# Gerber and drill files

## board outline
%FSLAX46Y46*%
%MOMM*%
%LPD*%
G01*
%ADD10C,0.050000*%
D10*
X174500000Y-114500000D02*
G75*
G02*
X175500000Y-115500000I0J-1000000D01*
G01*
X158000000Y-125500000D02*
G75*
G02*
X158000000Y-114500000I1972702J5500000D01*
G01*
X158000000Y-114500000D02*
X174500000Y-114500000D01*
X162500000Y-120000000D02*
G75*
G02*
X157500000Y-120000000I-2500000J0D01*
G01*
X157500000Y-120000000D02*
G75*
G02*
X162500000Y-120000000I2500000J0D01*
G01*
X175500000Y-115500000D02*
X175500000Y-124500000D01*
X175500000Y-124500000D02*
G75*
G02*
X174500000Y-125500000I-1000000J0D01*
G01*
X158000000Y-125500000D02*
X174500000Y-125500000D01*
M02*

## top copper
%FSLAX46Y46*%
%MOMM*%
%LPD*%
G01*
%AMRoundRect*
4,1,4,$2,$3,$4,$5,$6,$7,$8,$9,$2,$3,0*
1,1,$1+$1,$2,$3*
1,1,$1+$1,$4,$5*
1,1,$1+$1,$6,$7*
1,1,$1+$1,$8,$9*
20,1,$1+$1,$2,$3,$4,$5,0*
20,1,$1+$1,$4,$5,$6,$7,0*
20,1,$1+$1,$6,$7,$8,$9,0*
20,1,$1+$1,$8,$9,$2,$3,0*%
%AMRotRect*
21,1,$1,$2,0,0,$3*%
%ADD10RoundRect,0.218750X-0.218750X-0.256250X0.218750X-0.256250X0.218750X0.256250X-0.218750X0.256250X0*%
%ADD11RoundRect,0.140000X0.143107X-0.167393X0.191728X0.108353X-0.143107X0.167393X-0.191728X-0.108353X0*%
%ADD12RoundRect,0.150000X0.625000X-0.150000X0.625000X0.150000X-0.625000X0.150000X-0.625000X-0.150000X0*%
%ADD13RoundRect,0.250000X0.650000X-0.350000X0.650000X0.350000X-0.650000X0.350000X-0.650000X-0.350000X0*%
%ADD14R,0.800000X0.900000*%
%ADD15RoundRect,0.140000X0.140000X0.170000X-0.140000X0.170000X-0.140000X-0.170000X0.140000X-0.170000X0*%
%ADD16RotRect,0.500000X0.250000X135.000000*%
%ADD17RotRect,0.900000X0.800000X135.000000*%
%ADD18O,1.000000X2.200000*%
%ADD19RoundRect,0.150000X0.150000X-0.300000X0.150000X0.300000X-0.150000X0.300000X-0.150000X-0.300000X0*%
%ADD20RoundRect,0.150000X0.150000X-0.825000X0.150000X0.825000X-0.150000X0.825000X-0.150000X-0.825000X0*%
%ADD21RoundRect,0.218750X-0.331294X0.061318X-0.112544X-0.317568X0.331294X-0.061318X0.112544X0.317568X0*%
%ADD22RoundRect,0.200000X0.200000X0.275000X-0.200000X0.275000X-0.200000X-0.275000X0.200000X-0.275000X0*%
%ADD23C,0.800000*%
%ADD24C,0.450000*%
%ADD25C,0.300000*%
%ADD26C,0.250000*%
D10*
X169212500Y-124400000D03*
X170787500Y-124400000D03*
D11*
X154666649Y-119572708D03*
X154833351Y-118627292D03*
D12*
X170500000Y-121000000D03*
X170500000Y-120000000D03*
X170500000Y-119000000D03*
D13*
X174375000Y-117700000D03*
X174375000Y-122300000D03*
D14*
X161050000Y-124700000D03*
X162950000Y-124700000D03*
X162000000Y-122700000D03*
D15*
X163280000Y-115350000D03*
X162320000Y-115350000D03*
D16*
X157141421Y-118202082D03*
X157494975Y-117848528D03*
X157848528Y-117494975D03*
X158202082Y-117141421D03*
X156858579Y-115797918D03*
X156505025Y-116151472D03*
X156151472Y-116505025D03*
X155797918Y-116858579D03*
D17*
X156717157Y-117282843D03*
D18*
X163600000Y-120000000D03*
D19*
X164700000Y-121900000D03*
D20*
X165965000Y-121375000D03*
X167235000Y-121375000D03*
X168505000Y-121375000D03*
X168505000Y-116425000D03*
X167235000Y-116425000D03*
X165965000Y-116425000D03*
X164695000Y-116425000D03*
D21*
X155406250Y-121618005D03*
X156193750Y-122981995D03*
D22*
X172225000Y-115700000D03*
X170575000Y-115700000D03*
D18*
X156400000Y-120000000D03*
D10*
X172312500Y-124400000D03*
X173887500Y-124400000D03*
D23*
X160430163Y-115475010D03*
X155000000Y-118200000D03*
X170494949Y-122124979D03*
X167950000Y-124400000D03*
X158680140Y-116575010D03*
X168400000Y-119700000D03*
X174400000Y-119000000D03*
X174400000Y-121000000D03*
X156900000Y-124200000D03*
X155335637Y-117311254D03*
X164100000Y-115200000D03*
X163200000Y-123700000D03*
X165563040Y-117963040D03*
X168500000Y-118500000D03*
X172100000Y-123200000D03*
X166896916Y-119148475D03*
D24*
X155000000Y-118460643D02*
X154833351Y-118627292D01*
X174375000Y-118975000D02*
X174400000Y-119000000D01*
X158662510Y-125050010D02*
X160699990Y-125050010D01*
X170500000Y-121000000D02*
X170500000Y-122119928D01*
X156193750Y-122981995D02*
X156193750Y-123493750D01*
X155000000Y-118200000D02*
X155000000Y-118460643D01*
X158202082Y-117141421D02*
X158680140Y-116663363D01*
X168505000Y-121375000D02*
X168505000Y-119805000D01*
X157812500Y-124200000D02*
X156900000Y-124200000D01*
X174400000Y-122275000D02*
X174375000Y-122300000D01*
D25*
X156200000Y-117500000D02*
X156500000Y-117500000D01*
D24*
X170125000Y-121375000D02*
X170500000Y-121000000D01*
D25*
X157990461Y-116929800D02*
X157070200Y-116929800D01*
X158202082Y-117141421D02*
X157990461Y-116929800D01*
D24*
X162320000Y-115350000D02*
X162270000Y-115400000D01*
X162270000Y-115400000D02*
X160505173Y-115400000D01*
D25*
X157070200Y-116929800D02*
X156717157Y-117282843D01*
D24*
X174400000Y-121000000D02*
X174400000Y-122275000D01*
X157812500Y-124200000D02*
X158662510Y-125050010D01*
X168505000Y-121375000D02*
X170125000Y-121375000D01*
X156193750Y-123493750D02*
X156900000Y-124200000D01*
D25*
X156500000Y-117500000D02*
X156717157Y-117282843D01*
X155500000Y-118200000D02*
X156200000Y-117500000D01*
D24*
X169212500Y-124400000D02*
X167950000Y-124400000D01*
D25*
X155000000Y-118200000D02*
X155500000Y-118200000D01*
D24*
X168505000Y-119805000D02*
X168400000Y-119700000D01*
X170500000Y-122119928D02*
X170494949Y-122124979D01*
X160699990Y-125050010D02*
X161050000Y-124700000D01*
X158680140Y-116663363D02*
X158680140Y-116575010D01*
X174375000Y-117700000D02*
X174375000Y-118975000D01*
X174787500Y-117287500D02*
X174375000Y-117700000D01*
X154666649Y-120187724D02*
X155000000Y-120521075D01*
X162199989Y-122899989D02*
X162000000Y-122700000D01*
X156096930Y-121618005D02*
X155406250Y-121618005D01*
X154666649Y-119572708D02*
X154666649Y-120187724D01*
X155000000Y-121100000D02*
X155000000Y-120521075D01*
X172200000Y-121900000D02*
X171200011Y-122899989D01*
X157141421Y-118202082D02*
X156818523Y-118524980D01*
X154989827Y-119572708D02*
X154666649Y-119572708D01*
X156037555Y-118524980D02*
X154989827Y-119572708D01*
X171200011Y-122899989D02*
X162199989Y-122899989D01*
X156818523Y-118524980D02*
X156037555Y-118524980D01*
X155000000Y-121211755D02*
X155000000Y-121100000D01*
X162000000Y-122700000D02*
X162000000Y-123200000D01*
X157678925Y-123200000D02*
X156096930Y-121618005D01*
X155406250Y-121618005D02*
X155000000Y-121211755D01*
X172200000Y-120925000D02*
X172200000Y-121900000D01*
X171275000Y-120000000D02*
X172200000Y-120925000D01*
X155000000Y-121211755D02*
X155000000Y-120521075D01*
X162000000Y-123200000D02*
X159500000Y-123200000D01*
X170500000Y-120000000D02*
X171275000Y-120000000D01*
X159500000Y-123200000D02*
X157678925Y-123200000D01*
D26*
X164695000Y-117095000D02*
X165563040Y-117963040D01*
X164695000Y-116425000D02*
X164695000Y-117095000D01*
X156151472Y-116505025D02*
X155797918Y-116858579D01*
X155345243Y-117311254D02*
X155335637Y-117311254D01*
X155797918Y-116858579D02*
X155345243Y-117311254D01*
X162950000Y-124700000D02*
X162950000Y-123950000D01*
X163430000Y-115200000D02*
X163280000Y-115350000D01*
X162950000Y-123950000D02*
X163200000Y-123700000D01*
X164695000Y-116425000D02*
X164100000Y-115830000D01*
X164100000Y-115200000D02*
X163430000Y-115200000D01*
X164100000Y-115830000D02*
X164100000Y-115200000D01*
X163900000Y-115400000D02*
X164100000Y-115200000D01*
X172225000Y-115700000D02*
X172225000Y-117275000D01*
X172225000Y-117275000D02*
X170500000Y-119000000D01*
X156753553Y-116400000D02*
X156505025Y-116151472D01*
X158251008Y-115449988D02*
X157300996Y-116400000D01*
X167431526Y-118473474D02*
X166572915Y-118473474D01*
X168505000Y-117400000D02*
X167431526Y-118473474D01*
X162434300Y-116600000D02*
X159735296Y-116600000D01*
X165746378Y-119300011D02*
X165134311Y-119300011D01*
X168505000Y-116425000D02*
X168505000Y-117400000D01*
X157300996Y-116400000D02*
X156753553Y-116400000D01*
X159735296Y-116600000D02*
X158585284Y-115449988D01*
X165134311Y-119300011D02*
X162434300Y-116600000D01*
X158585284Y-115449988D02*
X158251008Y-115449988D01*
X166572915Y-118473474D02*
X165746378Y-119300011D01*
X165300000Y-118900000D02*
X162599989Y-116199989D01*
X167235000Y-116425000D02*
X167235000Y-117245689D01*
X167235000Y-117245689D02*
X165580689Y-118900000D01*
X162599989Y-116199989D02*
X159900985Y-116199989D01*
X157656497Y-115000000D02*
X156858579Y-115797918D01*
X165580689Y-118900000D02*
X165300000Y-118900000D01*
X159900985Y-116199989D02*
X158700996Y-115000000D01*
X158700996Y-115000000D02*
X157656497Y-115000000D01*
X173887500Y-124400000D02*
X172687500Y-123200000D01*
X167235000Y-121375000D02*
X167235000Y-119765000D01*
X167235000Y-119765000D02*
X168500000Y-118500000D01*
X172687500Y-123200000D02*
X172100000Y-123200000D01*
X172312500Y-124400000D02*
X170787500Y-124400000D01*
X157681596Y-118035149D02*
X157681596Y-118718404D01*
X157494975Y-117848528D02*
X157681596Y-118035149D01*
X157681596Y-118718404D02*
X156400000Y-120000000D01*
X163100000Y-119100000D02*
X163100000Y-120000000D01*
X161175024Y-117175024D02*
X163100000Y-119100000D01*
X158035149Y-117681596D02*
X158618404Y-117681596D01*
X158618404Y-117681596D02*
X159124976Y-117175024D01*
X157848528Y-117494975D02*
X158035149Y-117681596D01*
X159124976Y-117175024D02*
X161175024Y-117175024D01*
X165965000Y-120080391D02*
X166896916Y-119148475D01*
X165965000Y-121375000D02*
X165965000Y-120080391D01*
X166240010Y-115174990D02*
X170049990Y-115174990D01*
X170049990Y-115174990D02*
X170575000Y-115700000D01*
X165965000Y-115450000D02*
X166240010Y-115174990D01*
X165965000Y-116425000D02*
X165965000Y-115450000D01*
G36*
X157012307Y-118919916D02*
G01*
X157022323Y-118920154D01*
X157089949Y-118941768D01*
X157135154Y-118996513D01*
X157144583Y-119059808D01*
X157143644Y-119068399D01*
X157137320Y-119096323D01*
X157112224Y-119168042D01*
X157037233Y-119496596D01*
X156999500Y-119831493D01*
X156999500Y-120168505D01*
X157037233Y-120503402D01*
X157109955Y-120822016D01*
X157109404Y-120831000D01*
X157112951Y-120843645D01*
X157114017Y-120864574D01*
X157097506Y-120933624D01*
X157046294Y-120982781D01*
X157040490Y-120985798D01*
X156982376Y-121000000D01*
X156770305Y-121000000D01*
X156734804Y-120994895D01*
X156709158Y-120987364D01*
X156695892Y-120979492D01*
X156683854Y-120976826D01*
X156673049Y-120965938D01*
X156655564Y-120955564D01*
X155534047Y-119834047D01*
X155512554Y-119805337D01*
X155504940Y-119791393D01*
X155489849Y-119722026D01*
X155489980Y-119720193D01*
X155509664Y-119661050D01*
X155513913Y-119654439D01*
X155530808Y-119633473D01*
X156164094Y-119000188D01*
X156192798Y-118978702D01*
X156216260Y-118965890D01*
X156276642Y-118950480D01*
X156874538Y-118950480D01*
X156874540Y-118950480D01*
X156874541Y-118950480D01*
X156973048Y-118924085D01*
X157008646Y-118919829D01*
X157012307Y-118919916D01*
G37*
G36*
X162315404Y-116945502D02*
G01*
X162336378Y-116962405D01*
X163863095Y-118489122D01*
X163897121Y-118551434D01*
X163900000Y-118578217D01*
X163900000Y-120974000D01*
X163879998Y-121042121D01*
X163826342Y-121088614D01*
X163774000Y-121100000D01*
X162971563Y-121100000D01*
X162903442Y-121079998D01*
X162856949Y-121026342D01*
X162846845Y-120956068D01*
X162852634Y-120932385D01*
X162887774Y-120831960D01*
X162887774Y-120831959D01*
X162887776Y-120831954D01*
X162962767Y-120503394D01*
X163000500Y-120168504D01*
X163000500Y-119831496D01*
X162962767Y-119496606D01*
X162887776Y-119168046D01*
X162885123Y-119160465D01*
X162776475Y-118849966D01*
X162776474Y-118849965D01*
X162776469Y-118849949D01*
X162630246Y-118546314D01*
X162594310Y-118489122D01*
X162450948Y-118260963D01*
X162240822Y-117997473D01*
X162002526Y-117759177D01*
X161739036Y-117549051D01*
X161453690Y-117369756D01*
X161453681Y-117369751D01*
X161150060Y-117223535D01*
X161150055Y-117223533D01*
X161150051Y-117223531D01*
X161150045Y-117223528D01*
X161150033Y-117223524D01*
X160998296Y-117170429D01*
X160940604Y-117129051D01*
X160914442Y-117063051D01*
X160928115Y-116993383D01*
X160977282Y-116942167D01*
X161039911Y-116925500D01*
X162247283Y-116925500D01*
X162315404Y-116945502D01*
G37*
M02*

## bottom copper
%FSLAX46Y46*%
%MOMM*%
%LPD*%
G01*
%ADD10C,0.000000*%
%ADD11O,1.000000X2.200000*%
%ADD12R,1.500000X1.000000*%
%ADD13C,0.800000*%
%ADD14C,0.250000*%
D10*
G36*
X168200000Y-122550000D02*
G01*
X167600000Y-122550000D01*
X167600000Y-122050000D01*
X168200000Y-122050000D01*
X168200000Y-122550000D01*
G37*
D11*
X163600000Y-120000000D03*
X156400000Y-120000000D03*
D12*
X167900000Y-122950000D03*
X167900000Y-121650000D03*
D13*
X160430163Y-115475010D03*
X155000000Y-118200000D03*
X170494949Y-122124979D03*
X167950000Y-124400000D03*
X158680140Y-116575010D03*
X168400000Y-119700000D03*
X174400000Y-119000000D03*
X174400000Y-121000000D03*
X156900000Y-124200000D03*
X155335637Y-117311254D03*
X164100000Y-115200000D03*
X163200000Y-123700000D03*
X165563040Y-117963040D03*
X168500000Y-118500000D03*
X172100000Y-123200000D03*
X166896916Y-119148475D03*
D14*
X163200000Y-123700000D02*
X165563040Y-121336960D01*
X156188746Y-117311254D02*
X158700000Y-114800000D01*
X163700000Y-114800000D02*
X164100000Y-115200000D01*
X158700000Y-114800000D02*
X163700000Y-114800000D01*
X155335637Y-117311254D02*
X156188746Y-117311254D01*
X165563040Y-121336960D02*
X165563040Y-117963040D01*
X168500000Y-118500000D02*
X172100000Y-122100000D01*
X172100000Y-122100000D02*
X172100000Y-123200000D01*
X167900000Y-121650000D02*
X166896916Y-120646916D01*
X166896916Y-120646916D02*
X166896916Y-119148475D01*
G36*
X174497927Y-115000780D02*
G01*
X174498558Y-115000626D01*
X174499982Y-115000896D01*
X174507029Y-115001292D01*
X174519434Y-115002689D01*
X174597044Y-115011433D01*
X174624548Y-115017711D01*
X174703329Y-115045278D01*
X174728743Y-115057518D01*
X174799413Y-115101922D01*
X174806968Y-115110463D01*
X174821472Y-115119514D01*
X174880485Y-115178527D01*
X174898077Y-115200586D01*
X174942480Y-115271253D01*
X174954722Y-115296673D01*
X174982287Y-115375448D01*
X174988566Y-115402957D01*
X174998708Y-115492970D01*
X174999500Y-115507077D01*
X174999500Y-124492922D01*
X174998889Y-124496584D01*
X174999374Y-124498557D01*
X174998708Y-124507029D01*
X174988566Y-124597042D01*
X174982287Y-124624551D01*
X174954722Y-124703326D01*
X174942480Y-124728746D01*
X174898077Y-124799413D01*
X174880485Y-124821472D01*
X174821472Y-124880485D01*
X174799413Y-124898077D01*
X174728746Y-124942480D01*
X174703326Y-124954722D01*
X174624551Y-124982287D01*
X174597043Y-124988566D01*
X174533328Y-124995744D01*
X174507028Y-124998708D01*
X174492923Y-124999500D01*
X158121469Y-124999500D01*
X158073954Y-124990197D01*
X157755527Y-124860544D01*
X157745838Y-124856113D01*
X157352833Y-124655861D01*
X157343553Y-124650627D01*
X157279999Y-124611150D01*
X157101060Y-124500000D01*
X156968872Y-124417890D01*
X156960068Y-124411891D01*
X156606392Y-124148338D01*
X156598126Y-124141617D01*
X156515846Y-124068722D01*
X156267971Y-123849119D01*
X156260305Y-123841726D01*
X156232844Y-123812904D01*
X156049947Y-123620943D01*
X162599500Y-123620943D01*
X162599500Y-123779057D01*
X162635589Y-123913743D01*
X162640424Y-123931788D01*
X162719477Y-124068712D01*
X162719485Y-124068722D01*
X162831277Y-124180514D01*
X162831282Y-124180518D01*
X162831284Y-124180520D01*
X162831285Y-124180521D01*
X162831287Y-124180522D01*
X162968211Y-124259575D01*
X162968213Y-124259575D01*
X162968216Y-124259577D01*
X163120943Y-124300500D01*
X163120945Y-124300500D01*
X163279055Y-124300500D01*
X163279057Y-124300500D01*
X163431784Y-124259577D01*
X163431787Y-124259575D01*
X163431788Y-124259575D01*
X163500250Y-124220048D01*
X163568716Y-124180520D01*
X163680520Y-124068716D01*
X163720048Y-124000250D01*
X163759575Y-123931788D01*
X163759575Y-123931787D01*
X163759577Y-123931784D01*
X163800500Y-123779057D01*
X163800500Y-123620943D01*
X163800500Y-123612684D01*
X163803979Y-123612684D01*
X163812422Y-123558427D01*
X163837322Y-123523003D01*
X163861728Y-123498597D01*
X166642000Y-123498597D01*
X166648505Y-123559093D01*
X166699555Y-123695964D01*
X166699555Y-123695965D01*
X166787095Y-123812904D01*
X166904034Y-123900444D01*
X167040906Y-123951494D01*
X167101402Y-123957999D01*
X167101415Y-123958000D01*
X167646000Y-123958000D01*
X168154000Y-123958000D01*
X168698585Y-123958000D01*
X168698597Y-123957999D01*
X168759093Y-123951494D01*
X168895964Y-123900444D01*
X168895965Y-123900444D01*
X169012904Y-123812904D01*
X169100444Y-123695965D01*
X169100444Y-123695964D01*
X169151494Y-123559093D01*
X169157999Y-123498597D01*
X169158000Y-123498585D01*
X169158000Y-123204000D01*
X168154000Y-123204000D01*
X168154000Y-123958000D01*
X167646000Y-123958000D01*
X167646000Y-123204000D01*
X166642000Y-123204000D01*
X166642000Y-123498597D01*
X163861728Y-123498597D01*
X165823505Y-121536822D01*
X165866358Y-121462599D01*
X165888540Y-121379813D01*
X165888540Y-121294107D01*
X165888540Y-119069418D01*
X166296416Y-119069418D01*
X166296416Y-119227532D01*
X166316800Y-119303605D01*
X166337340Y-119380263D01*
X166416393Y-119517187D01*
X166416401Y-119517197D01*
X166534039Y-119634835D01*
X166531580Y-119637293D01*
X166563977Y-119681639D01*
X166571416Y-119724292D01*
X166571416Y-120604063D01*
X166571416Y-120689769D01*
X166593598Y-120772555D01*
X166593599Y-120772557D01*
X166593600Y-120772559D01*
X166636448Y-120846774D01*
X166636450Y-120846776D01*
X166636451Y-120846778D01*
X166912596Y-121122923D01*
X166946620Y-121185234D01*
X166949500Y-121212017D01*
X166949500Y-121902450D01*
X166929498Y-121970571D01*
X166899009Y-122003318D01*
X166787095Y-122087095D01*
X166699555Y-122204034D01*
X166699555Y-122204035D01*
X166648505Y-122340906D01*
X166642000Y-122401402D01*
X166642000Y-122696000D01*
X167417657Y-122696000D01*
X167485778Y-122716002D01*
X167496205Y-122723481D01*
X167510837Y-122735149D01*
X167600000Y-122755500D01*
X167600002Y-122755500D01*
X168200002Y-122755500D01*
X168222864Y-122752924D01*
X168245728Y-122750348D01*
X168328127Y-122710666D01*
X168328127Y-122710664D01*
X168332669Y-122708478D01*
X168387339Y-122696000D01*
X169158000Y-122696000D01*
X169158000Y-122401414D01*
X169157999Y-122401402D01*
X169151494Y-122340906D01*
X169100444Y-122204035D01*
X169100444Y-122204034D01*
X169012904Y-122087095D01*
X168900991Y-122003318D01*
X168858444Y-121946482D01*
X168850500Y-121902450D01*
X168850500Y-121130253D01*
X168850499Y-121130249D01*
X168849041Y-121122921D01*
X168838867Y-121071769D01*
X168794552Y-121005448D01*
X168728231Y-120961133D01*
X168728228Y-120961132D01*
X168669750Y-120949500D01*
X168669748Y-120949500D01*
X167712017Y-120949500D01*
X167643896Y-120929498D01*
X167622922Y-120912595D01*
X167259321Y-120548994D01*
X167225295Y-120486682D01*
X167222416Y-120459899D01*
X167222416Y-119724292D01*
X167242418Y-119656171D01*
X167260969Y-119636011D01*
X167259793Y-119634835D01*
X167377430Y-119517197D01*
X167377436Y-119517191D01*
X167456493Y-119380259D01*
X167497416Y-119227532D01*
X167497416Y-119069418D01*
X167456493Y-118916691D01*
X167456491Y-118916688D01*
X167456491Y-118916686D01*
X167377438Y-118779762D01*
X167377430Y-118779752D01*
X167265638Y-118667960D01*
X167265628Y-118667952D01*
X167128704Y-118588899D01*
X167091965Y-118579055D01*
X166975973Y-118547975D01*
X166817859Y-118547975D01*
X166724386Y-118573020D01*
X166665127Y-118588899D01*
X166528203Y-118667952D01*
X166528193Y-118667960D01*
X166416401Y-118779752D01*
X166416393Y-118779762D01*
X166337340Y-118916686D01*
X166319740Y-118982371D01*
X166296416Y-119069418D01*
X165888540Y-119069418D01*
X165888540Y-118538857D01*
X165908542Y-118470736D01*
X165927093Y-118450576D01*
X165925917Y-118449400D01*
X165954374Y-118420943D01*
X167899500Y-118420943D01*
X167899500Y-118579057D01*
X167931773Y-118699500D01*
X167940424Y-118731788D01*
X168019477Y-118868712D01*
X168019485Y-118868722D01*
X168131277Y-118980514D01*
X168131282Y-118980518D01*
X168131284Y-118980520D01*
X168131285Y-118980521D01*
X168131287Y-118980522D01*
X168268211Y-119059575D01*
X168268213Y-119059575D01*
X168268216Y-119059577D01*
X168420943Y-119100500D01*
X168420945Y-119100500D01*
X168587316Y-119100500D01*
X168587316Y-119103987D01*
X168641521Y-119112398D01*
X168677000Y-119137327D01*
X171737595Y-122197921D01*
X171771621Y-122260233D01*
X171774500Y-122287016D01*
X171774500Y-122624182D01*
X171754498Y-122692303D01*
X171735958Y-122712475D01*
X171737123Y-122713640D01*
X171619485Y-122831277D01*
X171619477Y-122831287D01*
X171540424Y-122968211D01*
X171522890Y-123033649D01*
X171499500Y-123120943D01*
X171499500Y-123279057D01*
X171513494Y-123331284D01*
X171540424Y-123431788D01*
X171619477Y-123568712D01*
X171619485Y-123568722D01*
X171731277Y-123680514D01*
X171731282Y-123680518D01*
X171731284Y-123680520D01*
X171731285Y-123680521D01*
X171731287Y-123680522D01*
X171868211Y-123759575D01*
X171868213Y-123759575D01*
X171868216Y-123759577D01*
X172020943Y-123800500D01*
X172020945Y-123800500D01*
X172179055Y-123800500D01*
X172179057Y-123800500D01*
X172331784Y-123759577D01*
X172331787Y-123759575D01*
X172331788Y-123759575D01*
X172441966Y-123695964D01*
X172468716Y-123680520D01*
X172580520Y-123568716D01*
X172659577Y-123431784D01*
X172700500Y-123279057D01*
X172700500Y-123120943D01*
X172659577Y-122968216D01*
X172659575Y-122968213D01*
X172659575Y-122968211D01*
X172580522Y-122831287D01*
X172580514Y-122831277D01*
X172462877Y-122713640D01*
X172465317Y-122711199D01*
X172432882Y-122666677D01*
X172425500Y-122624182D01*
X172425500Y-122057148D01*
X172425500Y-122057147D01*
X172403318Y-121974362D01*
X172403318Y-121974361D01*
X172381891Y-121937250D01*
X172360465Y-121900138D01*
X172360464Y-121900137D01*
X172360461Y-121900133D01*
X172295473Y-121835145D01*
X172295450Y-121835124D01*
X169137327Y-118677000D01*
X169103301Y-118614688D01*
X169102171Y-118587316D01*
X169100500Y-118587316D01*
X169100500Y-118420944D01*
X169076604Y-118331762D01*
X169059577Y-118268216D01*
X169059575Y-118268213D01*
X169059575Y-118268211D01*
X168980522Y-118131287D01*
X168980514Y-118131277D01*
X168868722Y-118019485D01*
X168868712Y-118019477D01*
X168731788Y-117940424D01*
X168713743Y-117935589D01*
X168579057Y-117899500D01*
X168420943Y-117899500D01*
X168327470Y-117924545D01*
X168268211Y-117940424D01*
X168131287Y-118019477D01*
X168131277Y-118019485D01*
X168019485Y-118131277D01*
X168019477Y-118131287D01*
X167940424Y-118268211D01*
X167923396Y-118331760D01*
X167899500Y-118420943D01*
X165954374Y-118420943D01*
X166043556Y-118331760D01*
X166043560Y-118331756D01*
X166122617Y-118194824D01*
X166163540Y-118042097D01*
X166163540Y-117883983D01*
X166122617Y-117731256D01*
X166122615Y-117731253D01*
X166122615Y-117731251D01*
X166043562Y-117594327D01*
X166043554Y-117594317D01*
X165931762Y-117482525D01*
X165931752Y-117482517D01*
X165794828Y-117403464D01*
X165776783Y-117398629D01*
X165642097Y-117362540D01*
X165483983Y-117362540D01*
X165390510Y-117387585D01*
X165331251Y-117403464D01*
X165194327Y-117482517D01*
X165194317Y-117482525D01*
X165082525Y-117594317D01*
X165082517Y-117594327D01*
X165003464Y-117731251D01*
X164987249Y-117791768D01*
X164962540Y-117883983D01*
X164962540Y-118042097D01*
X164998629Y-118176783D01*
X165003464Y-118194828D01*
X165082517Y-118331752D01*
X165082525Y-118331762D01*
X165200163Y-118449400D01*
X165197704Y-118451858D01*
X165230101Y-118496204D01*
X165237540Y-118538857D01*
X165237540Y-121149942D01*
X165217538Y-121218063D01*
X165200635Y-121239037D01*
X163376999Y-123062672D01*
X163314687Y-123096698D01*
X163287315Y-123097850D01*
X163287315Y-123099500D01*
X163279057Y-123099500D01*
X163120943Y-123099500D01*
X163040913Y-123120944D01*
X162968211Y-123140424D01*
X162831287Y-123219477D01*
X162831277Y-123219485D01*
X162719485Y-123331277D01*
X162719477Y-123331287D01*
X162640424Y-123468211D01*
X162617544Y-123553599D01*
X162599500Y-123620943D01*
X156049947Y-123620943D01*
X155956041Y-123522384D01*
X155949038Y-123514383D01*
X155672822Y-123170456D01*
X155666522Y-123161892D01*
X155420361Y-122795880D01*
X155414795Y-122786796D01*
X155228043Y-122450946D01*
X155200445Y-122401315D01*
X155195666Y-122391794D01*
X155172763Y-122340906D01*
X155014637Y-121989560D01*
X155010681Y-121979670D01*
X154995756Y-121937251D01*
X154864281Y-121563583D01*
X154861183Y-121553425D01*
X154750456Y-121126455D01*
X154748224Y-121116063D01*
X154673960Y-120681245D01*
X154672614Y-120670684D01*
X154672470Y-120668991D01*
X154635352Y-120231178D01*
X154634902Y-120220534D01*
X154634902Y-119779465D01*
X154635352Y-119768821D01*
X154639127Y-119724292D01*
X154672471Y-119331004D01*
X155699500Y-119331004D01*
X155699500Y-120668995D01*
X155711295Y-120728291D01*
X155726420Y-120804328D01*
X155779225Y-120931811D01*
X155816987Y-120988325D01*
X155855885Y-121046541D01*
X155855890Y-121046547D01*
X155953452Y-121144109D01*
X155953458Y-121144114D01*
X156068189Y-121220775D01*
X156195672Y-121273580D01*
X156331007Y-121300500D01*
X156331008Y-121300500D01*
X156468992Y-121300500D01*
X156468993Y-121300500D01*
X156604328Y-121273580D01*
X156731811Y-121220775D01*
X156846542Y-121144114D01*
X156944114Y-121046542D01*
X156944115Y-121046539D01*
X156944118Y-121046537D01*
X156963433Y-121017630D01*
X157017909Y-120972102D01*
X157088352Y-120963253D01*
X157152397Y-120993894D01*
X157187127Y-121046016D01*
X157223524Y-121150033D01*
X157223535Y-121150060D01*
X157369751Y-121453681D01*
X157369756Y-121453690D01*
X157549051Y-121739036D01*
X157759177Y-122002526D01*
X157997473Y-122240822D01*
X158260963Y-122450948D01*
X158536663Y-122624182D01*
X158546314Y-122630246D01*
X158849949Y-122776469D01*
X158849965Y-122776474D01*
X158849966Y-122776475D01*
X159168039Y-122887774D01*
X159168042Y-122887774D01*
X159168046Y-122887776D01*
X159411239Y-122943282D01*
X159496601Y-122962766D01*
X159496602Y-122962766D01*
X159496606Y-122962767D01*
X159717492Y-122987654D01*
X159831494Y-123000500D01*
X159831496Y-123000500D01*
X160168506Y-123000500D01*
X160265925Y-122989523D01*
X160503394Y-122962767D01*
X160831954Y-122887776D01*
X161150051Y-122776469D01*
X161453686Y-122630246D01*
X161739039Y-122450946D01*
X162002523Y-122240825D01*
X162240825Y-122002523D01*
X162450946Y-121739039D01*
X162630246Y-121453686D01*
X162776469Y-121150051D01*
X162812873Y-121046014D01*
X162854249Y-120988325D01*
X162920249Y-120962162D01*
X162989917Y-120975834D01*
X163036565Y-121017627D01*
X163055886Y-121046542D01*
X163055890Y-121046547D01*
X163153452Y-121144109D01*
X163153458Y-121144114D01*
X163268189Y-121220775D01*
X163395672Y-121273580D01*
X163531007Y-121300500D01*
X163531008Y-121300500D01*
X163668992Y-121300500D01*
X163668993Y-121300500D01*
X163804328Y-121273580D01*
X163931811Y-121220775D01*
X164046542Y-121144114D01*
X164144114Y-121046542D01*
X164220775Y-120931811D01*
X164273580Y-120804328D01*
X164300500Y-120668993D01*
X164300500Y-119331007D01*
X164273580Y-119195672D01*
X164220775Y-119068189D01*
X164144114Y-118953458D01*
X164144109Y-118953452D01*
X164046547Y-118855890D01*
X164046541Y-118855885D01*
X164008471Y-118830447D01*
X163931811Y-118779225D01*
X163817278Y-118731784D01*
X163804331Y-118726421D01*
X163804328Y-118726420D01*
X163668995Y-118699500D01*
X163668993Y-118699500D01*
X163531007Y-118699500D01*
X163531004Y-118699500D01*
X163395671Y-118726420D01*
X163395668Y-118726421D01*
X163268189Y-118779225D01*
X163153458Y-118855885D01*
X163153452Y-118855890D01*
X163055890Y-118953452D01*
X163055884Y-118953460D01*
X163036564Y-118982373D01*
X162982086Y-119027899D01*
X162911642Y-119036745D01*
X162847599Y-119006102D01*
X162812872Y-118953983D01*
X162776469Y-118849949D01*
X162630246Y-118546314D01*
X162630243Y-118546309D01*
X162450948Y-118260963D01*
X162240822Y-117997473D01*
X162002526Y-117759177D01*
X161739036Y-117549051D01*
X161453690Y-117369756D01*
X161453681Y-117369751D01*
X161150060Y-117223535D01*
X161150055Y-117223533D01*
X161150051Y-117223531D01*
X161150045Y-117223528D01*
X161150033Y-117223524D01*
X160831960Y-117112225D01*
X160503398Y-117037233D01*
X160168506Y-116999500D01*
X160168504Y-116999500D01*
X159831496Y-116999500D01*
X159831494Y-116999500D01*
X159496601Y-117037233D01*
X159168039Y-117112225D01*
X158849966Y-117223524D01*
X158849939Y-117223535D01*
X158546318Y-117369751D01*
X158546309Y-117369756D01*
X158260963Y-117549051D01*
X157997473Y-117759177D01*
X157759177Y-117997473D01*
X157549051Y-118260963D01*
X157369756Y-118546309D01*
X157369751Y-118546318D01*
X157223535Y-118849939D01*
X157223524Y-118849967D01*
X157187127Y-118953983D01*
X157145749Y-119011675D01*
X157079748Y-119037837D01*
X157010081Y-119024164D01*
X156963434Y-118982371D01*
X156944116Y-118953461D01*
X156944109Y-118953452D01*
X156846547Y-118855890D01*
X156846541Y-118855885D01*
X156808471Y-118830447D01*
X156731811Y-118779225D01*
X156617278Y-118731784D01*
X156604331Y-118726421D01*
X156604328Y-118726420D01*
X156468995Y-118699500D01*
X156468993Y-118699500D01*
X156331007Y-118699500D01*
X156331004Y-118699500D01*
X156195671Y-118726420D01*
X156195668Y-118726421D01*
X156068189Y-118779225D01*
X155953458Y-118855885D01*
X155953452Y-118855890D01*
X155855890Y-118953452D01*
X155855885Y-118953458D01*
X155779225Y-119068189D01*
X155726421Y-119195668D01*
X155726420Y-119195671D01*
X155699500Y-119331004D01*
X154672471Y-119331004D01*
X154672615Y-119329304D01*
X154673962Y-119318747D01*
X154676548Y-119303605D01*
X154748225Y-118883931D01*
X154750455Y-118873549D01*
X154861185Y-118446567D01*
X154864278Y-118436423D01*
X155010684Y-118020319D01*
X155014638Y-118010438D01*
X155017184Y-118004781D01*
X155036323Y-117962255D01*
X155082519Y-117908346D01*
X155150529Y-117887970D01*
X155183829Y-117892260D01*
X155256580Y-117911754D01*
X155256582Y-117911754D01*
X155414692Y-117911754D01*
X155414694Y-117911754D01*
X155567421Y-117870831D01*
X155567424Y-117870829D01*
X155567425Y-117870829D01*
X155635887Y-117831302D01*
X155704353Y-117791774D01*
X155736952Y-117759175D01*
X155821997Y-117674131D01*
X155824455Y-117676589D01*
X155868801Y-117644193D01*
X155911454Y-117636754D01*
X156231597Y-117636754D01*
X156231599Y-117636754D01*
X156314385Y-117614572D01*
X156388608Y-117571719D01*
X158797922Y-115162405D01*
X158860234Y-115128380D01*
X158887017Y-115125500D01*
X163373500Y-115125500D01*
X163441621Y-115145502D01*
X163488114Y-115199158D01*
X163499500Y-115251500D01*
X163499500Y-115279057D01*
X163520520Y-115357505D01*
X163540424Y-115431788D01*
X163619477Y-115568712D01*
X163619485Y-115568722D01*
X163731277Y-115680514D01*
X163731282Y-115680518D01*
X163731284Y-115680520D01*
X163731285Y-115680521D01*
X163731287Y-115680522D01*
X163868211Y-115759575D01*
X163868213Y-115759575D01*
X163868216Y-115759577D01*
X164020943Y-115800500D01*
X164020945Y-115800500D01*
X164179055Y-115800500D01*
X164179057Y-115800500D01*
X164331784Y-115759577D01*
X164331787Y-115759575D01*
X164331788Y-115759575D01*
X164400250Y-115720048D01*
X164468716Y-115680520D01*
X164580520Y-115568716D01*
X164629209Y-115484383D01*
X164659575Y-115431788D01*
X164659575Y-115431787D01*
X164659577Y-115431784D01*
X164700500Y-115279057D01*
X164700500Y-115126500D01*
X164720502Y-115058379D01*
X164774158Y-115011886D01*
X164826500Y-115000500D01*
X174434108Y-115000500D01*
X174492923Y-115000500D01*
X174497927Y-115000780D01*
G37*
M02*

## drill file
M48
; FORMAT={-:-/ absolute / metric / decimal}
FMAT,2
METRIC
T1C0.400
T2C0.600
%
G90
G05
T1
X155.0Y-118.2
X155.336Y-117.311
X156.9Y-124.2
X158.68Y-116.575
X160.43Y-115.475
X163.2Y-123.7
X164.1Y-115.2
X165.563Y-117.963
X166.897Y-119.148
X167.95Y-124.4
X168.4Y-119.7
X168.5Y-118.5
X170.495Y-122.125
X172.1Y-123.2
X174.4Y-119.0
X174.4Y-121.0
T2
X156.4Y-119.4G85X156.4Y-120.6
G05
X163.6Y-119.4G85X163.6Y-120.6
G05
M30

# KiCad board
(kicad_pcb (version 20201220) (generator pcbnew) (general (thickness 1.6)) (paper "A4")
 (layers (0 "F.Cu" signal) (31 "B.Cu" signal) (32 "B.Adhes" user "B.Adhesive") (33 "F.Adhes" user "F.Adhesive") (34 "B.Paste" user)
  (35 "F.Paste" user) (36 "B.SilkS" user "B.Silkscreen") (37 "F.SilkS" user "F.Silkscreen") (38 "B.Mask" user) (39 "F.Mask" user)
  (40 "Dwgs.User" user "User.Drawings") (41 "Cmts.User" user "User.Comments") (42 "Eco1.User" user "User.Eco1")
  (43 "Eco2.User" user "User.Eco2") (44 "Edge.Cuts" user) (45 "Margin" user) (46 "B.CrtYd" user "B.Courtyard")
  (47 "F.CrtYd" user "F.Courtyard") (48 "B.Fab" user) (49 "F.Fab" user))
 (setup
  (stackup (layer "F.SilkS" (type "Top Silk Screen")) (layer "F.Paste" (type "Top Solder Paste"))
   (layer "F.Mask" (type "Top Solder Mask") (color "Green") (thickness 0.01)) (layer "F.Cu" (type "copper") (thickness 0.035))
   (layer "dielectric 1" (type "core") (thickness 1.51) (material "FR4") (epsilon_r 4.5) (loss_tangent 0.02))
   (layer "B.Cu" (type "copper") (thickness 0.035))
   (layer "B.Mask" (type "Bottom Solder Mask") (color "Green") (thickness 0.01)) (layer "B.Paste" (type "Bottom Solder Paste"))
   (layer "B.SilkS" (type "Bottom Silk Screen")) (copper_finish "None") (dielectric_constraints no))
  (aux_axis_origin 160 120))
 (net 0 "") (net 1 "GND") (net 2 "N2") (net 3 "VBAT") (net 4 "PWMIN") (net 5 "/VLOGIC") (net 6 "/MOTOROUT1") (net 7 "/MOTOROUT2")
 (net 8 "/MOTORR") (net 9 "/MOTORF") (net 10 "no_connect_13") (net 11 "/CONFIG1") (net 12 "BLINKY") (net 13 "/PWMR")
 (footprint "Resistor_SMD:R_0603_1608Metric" (layer "F.Cu") (at 170 124.4)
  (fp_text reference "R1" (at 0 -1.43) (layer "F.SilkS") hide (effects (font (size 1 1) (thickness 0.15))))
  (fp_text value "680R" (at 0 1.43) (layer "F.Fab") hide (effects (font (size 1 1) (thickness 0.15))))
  (pad "1" smd roundrect (at -0.7875 0) (size 0.875 0.95) (layers "F.Cu" "F.Paste" "F.Mask") (roundrect_rratio 0.25) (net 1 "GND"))
  (pad "2" smd roundrect (at 0.7875 0) (size 0.875 0.95) (layers "F.Cu" "F.Paste" "F.Mask") (roundrect_rratio 0.25) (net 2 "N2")))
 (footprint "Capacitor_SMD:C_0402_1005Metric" (layer "F.Cu") (at 154.75 119.1 80)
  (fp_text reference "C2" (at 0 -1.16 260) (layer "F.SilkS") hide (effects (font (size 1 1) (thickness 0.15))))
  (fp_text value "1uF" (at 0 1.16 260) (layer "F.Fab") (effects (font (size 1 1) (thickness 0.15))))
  (pad "1" smd roundrect (at -0.48 0 80) (size 0.56 0.62) (layers "F.Cu" "F.Paste" "F.Mask") (roundrect_rratio 0.25) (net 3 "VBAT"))
  (pad "2" smd roundrect (at 0.48 0 80) (size 0.56 0.62) (layers "F.Cu" "F.Paste" "F.Mask") (roundrect_rratio 0.25) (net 1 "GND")))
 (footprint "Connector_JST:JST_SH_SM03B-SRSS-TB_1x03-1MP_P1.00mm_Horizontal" (layer "F.Cu") (at 172.5 120 90)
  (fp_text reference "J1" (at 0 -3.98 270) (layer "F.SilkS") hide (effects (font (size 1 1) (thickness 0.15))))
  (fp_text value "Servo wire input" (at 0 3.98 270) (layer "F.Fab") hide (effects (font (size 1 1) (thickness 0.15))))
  (pad "1" smd roundrect (at -1 -2 90) (size 0.6 1.55) (layers "F.Cu" "F.Paste" "F.Mask") (roundrect_rratio 0.25) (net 1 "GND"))
  (pad "2" smd roundrect (at 0 -2 90) (size 0.6 1.55) (layers "F.Cu" "F.Paste" "F.Mask") (roundrect_rratio 0.25) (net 3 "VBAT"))
  (pad "3" smd roundrect (at 1 -2 90) (size 0.6 1.55) (layers "F.Cu" "F.Paste" "F.Mask") (roundrect_rratio 0.25) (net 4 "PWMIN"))
  (pad "MP" smd roundrect (at 2.3 1.875 90) (size 1.2 1.8) (layers "F.Cu" "F.Paste" "F.Mask") (roundrect_rratio 0.2083333333333333)
   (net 1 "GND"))
  (pad "MP" smd roundrect (at -2.3 1.875 90) (size 1.2 1.8) (layers "F.Cu" "F.Paste" "F.Mask") (roundrect_rratio 0.2083333333333333)
   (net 1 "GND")))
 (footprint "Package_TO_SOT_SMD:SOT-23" (layer "F.Cu") (at 162 123.7 90)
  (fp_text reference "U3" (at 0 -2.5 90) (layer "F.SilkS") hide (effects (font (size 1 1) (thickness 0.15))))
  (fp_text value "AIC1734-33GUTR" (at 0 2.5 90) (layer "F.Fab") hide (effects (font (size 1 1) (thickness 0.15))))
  (pad "1" smd rect (at -1 -0.95 90) (size 0.9 0.8) (layers "F.Cu" "F.Paste" "F.Mask") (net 1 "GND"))
  (pad "2" smd rect (at -1 0.95 90) (size 0.9 0.8) (layers "F.Cu" "F.Paste" "F.Mask") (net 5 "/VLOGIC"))
  (pad "3" smd rect (at 1 0 90) (size 0.9 0.8) (layers "F.Cu" "F.Paste" "F.Mask") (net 3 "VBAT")))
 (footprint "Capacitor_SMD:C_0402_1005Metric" (layer "F.Cu") (at 162.8 115.35 180)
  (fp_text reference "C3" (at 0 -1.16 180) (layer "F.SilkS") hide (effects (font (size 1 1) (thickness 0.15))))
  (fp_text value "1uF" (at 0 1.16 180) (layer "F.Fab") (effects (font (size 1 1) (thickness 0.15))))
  (pad "1" smd roundrect (at -0.48 0 180) (size 0.56 0.62) (layers "F.Cu" "F.Paste" "F.Mask") (roundrect_rratio 0.25) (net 5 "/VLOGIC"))
  (pad "2" smd roundrect (at 0.48 0 180) (size 0.56 0.62) (layers "F.Cu" "F.Paste" "F.Mask") (roundrect_rratio 0.25) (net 1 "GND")))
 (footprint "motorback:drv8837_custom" (layer "F.Cu") (at 157 117 135)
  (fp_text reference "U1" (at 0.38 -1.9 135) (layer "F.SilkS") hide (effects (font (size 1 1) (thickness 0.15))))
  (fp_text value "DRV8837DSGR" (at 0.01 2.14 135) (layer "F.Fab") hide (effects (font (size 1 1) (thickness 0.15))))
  (pad "" smd rect (at 0 -0.4 135) (size 0.75 0.65) (layers "F.Paste"))
  (pad "1" smd rect (at -0.95 -0.75 135) (size 0.5 0.25) (layers "F.Cu" "F.Paste" "F.Mask") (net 3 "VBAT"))
  (pad "2" smd rect (at -0.95 -0.25 135) (size 0.5 0.25) (layers "F.Cu" "F.Paste" "F.Mask") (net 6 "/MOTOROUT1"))
  (pad "3" smd rect (at -0.95 0.25 135) (size 0.5 0.25) (layers "F.Cu" "F.Paste" "F.Mask") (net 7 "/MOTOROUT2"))
  (pad "4" smd rect (at -0.95 0.75 135) (size 0.5 0.25) (layers "F.Cu" "F.Paste" "F.Mask") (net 1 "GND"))
  (pad "5" smd rect (at 0.95 0.75 135) (size 0.5 0.25) (layers "F.Cu" "F.Paste" "F.Mask") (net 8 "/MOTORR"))
  (pad "6" smd rect (at 0.95 0.25 135) (size 0.5 0.25) (layers "F.Cu" "F.Paste" "F.Mask") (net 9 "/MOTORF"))
  (pad "7" smd rect (at 0.95 -0.25 135) (size 0.5 0.25) (layers "F.Cu" "F.Paste" "F.Mask") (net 5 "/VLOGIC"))
  (pad "8" smd rect (at 0.95 -0.75 135) (size 0.5 0.25) (layers "F.Cu" "F.Paste" "F.Mask") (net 5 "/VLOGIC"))
  (pad "9" smd rect (at 0 -0.4 135) (size 0.9 0.8) (layers "F.Cu" "F.Mask") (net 1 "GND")))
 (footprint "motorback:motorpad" (layer "F.Cu") (at 163.6 120)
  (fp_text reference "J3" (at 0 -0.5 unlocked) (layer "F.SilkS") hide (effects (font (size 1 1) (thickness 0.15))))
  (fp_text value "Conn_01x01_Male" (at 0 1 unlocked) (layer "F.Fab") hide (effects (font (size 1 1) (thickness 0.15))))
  (pad "1" thru_hole oval (at 0 0) (size 1 2.2) (drill oval 0.6 1.8) (layers *.Cu *.Mask) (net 7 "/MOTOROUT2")))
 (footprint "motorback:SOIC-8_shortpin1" (layer "F.Cu") (at 166.6 118.9 90)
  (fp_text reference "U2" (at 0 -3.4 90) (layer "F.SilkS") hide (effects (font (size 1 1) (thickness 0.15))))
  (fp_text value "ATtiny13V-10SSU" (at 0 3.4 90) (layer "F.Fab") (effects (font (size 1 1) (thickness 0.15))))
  (pad "1" smd roundrect (at -3 -1.9 90) (size 0.9 0.6) (layers "F.Cu" "F.Paste" "F.Mask") (roundrect_rratio 0.25) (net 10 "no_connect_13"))
  (pad "2" smd roundrect (at -2.475 -0.635 90) (size 1.95 0.6) (layers "F.Cu" "F.Paste" "F.Mask") (roundrect_rratio 0.25)
   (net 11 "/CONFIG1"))
  (pad "3" smd roundrect (at -2.475 0.635 90) (size 1.95 0.6) (layers "F.Cu" "F.Paste" "F.Mask") (roundrect_rratio 0.25) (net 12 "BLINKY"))
  (pad "4" smd roundrect (at -2.475 1.905 90) (size 1.95 0.6) (layers "F.Cu" "F.Paste" "F.Mask") (roundrect_rratio 0.25) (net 1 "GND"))
  (pad "5" smd roundrect (at 2.475 1.905 90) (size 1.95 0.6) (layers "F.Cu" "F.Paste" "F.Mask") (roundrect_rratio 0.25) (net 9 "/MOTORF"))
  (pad "6" smd roundrect (at 2.475 0.635 90) (size 1.95 0.6) (layers "F.Cu" "F.Paste" "F.Mask") (roundrect_rratio 0.25) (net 8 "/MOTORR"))
  (pad "7" smd roundrect (at 2.475 -0.635 90) (size 1.95 0.6) (layers "F.Cu" "F.Paste" "F.Mask") (roundrect_rratio 0.25) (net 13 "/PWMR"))
  (pad "8" smd roundrect (at 2.475 -1.905 90) (size 1.95 0.6) (layers "F.Cu" "F.Paste" "F.Mask") (roundrect_rratio 0.25) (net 5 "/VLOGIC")))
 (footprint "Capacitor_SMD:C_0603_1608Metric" (layer "F.Cu") (at 155.8 122.3 -60)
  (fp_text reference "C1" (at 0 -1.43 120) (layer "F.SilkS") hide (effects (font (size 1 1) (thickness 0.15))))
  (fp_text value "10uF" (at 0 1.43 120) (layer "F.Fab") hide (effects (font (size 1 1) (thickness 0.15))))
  (pad "1" smd roundrect (at -0.7875 0 300) (size 0.875 0.95) (layers "F.Cu" "F.Paste" "F.Mask") (roundrect_rratio 0.25) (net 3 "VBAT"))
  (pad "2" smd roundrect (at 0.7875 0 300) (size 0.875 0.95) (layers "F.Cu" "F.Paste" "F.Mask") (roundrect_rratio 0.25) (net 1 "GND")))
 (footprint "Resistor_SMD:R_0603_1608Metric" (layer "F.Cu") (at 171.4 115.7 180)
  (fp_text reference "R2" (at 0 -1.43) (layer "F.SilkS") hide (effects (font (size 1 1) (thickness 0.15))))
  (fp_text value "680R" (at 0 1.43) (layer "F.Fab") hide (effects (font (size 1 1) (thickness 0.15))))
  (pad "1" smd roundrect (at -0.825 0 180) (size 0.8 0.95) (layers "F.Cu" "F.Paste" "F.Mask") (roundrect_rratio 0.25) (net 4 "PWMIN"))
  (pad "2" smd roundrect (at 0.825 0 180) (size 0.8 0.95) (layers "F.Cu" "F.Paste" "F.Mask") (roundrect_rratio 0.25) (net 13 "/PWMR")))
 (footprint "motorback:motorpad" (layer "F.Cu") (at 156.4 120)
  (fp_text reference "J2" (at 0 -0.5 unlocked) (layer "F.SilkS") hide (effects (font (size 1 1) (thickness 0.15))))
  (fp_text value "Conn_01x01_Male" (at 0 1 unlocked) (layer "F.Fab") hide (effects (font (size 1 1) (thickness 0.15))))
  (pad "1" thru_hole oval (at 0 0) (size 1 2.2) (drill oval 0.6 1.8) (layers *.Cu *.Mask) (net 6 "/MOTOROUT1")))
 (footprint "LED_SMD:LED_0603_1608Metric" (layer "F.Cu") (at 173.1 124.4)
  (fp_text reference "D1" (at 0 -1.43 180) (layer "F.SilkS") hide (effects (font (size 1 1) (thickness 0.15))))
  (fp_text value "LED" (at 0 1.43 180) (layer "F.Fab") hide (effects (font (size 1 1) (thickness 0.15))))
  (pad "1" smd roundrect (at -0.7875 0) (size 0.875 0.95) (layers "F.Cu" "F.Paste" "F.Mask") (roundrect_rratio 0.25) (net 2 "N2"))
  (pad "2" smd roundrect (at 0.7875 0) (size 0.875 0.95) (layers "F.Cu" "F.Paste" "F.Mask") (roundrect_rratio 0.25) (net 12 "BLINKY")))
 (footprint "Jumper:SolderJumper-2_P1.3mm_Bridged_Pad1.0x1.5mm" (layer "B.Cu") (at 167.9 122.3 90)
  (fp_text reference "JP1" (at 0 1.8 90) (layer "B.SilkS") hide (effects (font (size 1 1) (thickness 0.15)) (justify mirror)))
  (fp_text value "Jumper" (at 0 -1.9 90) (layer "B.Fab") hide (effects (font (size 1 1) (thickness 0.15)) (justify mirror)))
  (fp_poly (pts (xy -0.25 0.3) (xy 0.25 0.3) (xy 0.25 -0.3) (xy -0.25 -0.3)) (layer "B.Cu") (width 0) (fill solid))
  (pad "1" smd rect (at -0.65 0 90) (size 1 1.5) (layers "B.Cu" "B.Mask") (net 1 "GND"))
  (pad "2" smd rect (at 0.65 0 90) (size 1 1.5) (layers "B.Cu" "B.Mask") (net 11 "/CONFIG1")))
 (gr_arc (start 174.5 115.5) (end 175.5 115.5) (angle -90) (layer "Edge.Cuts") (width 0.05))
 (gr_arc (start 159.972702 120) (end 158 114.5) (angle -140.5369116) (layer "Edge.Cuts") (width 0.05))
 (gr_line (start 158 114.5) (end 174.5 114.5) (layer "Edge.Cuts") (width 0.05))
 (gr_circle (center 160 120) (end 162.5 120) (layer "Edge.Cuts") (width 0.05) (fill none))
 (gr_line (start 175.5 115.5) (end 175.5 124.5) (layer "Edge.Cuts") (width 0.05))
 (gr_arc (start 174.5 124.5) (end 174.5 125.5) (angle -90) (layer "Edge.Cuts") (width 0.05))
 (gr_line (start 158 125.5) (end 174.5 125.5) (layer "Edge.Cuts") (width 0.05))
 (segment (start 155 118.460643) (end 154.833351 118.627292) (width 0.45) (layer "F.Cu") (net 1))
 (segment (start 174.375 118.975) (end 174.4 119) (width 0.45) (layer "F.Cu") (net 1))
 (segment (start 158.66251 125.05001) (end 160.69999 125.05001) (width 0.45) (layer "F.Cu") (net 1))
 (segment (start 170.5 121) (end 170.5 122.119928) (width 0.45) (layer "F.Cu") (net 1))
 (segment (start 156.19375 122.981995) (end 156.19375 123.49375) (width 0.45) (layer "F.Cu") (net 1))
 (segment (start 155 118.2) (end 155 118.460643) (width 0.45) (layer "F.Cu") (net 1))
 (segment (start 158.202082 117.141421) (end 158.68014 116.663363) (width 0.45) (layer "F.Cu") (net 1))
 (segment (start 168.505 121.375) (end 168.505 119.805) (width 0.45) (layer "F.Cu") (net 1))
 (segment (start 157.8125 124.2) (end 156.9 124.2) (width 0.45) (layer "F.Cu") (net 1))
 (segment (start 174.4 122.275) (end 174.375 122.3) (width 0.45) (layer "F.Cu") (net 1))
 (segment (start 156.2 117.5) (end 156.5 117.5) (width 0.3) (layer "F.Cu") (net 1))
 (segment (start 170.125 121.375) (end 170.5 121) (width 0.45) (layer "F.Cu") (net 1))
 (segment (start 157.990461 116.9298) (end 157.0702 116.9298) (width 0.3) (layer "F.Cu") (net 1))
 (segment (start 158.202082 117.141421) (end 157.990461 116.9298) (width 0.3) (layer "F.Cu") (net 1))
 (segment (start 162.32 115.35) (end 162.27 115.4) (width 0.45) (layer "F.Cu") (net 1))
 (segment (start 162.27 115.4) (end 160.505173 115.4) (width 0.45) (layer "F.Cu") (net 1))
 (segment (start 157.0702 116.9298) (end 156.717157 117.282843) (width 0.3) (layer "F.Cu") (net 1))
 (segment (start 174.4 121) (end 174.4 122.275) (width 0.45) (layer "F.Cu") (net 1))
 (segment (start 157.8125 124.2) (end 158.66251 125.05001) (width 0.45) (layer "F.Cu") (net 1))
 (segment (start 168.505 121.375) (end 170.125 121.375) (width 0.45) (layer "F.Cu") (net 1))
 (segment (start 156.19375 123.49375) (end 156.9 124.2) (width 0.45) (layer "F.Cu") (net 1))
 (segment (start 156.5 117.5) (end 156.717157 117.282843) (width 0.3) (layer "F.Cu") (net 1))
 (segment (start 155.5 118.2) (end 156.2 117.5) (width 0.3) (layer "F.Cu") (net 1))
 (segment (start 169.2125 124.4) (end 167.95 124.4) (width 0.45) (layer "F.Cu") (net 1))
 (segment (start 155 118.2) (end 155.5 118.2) (width 0.3) (layer "F.Cu") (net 1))
 (segment (start 168.505 119.805) (end 168.4 119.7) (width 0.45) (layer "F.Cu") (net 1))
 (segment (start 170.5 122.119928) (end 170.494949 122.124979) (width 0.45) (layer "F.Cu") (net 1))
 (segment (start 160.69999 125.05001) (end 161.05 124.7) (width 0.45) (layer "F.Cu") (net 1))
 (segment (start 158.68014 116.663363) (end 158.68014 116.57501) (width 0.45) (layer "F.Cu") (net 1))
 (segment (start 174.375 117.7) (end 174.375 118.975) (width 0.45) (layer "F.Cu") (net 1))
 (segment (start 174.7875 117.2875) (end 174.375 117.7) (width 0.45) (layer "F.Cu") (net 1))
 (via (at 160.430163 115.47501) (size 0.8) (drill 0.4) (layers "F.Cu" "B.Cu") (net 1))
 (via (at 155 118.2) (size 0.8) (drill 0.4) (layers "F.Cu" "B.Cu") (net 1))
 (via (at 170.494949 122.124979) (size 0.8) (drill 0.4) (layers "F.Cu" "B.Cu") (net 1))
 (via (at 167.95 124.4) (size 0.8) (drill 0.4) (layers "F.Cu" "B.Cu") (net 1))
 (via (at 158.68014 116.57501) (size 0.8) (drill 0.4) (layers "F.Cu" "B.Cu") (free) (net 1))
 (via (at 168.4 119.7) (size 0.8) (drill 0.4) (layers "F.Cu" "B.Cu") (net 1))
 (via (at 174.4 119) (size 0.8) (drill 0.4) (layers "F.Cu" "B.Cu") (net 1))
 (via (at 174.4 121) (size 0.8) (drill 0.4) (layers "F.Cu" "B.Cu") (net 1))
 (via (at 156.9 124.2) (size 0.8) (drill 0.4) (layers "F.Cu" "B.Cu") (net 1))
 (segment (start 154.666649 120.187724) (end 155 120.521075) (width 0.45) (layer "F.Cu") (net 3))
 (segment (start 162.199989 122.899989) (end 162 122.7) (width 0.45) (layer "F.Cu") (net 3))
 (segment (start 156.09693 121.618005) (end 155.40625 121.618005) (width 0.45) (layer "F.Cu") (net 3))
 (segment (start 154.666649 119.572708) (end 154.666649 120.187724) (width 0.45) (layer "F.Cu") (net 3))
 (segment (start 155 121.1) (end 155 120.521075) (width 0.45) (layer "F.Cu") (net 3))
 (segment (start 172.2 121.9) (end 171.200011 122.899989) (width 0.45) (layer "F.Cu") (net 3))
 (segment (start 157.141421 118.202082) (end 156.818523 118.52498) (width 0.45) (layer "F.Cu") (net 3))
 (segment (start 154.989827 119.572708) (end 154.666649 119.572708) (width 0.45) (layer "F.Cu") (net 3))
 (segment (start 156.037555 118.52498) (end 154.989827 119.572708) (width 0.45) (layer "F.Cu") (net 3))
 (segment (start 171.200011 122.899989) (end 162.199989 122.899989) (width 0.45) (layer "F.Cu") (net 3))
 (segment (start 156.818523 118.52498) (end 156.037555 118.52498) (width 0.45) (layer "F.Cu") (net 3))
 (segment (start 155 121.211755) (end 155 121.1) (width 0.45) (layer "F.Cu") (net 3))
 (segment (start 162 122.7) (end 162 123.2) (width 0.45) (layer "F.Cu") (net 3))
 (segment (start 157.678925 123.2) (end 156.09693 121.618005) (width 0.45) (layer "F.Cu") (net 3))
 (segment (start 155.40625 121.618005) (end 155 121.211755) (width 0.45) (layer "F.Cu") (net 3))
 (segment (start 172.2 120.925) (end 172.2 121.9) (width 0.45) (layer "F.Cu") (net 3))
 (segment (start 171.275 120) (end 172.2 120.925) (width 0.45) (layer "F.Cu") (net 3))
 (segment (start 155 121.211755) (end 155 120.521075) (width 0.45) (layer "F.Cu") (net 3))
 (segment (start 162 123.2) (end 159.5 123.2) (width 0.45) (layer "F.Cu") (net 3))
 (segment (start 170.5 120) (end 171.275 120) (width 0.45) (layer "F.Cu") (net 3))
 (segment (start 159.5 123.2) (end 157.678925 123.2) (width 0.45) (layer "F.Cu") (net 3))
 (segment (start 164.695 117.095) (end 165.56304 117.96304) (width 0.25) (layer "F.Cu") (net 5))
 (segment (start 164.695 116.425) (end 164.695 117.095) (width 0.25) (layer "F.Cu") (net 5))
 (segment (start 156.151472 116.505025) (end 155.797918 116.858579) (width 0.25) (layer "F.Cu") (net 5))
 (segment (start 155.345243 117.311254) (end 155.335637 117.311254) (width 0.25) (layer "F.Cu") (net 5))
 (segment (start 155.797918 116.858579) (end 155.345243 117.311254) (width 0.25) (layer "F.Cu") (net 5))
 (segment (start 162.95 124.7) (end 162.95 123.95) (width 0.25) (layer "F.Cu") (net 5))
 (segment (start 163.43 115.2) (end 163.28 115.35) (width 0.25) (layer "F.Cu") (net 5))
 (segment (start 162.95 123.95) (end 163.2 123.7) (width 0.25) (layer "F.Cu") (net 5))
 (segment (start 164.695 116.425) (end 164.1 115.83) (width 0.25) (layer "F.Cu") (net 5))
 (segment (start 164.1 115.2) (end 163.43 115.2) (width 0.25) (layer "F.Cu") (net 5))
 (segment (start 164.1 115.83) (end 164.1 115.2) (width 0.25) (layer "F.Cu") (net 5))
 (segment (start 163.9 115.4) (end 164.1 115.2) (width 0.25) (layer "F.Cu") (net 5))
 (via (at 155.335637 117.311254) (size 0.8) (drill 0.4) (layers "F.Cu" "B.Cu") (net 5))
 (via (at 164.1 115.2) (size 0.8) (drill 0.4) (layers "F.Cu" "B.Cu") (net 5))
 (via (at 163.2 123.7) (size 0.8) (drill 0.4) (layers "F.Cu" "B.Cu") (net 5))
 (via (at 165.56304 117.96304) (size 0.8) (drill 0.4) (layers "F.Cu" "B.Cu") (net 5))
 (segment (start 163.2 123.7) (end 165.56304 121.33696) (width 0.25) (layer "B.Cu") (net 5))
 (segment (start 156.188746 117.311254) (end 158.7 114.8) (width 0.25) (layer "B.Cu") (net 5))
 (segment (start 163.7 114.8) (end 164.1 115.2) (width 0.25) (layer "B.Cu") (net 5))
 (segment (start 158.7 114.8) (end 163.7 114.8) (width 0.25) (layer "B.Cu") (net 5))
 (segment (start 155.335637 117.311254) (end 156.188746 117.311254) (width 0.25) (layer "B.Cu") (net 5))
 (segment (start 165.56304 121.33696) (end 165.56304 117.96304) (width 0.25) (layer "B.Cu") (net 5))
 (segment (start 172.225 115.7) (end 172.225 117.275) (width 0.25) (layer "F.Cu") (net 4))
 (segment (start 172.225 117.275) (end 170.5 119) (width 0.25) (layer "F.Cu") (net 4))
 (segment (start 156.753553 116.4) (end 156.505025 116.151472) (width 0.25) (layer "F.Cu") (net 9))
 (segment (start 158.251008 115.449988) (end 157.300996 116.4) (width 0.25) (layer "F.Cu") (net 9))
 (segment (start 167.431526 118.473474) (end 166.572915 118.473474) (width 0.25) (layer "F.Cu") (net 9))
 (segment (start 168.505 117.4) (end 167.431526 118.473474) (width 0.25) (layer "F.Cu") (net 9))
 (segment (start 162.4343 116.6) (end 159.735296 116.6) (width 0.25) (layer "F.Cu") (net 9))
 (segment (start 165.746378 119.300011) (end 165.134311 119.300011) (width 0.25) (layer "F.Cu") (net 9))
 (segment (start 168.505 116.425) (end 168.505 117.4) (width 0.25) (layer "F.Cu") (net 9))
 (segment (start 157.300996 116.4) (end 156.753553 116.4) (width 0.25) (layer "F.Cu") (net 9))
 (segment (start 159.735296 116.6) (end 158.585284 115.449988) (width 0.25) (layer "F.Cu") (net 9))
 (segment (start 165.134311 119.300011) (end 162.4343 116.6) (width 0.25) (layer "F.Cu") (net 9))
 (segment (start 158.585284 115.449988) (end 158.251008 115.449988) (width 0.25) (layer "F.Cu") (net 9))
 (segment (start 166.572915 118.473474) (end 165.746378 119.300011) (width 0.25) (layer "F.Cu") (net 9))
 (segment (start 165.3 118.9) (end 162.599989 116.199989) (width 0.25) (layer "F.Cu") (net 8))
 (segment (start 167.235 116.425) (end 167.235 117.245689) (width 0.25) (layer "F.Cu") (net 8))
 (segment (start 167.235 117.245689) (end 165.580689 118.9) (width 0.25) (layer "F.Cu") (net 8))
 (segment (start 162.599989 116.199989) (end 159.900985 116.199989) (width 0.25) (layer "F.Cu") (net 8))
 (segment (start 157.656497 115) (end 156.858579 115.797918) (width 0.25) (layer "F.Cu") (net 8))
 (segment (start 165.580689 118.9) (end 165.3 118.9) (width 0.25) (layer "F.Cu") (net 8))
 (segment (start 159.900985 116.199989) (end 158.700996 115) (width 0.25) (layer "F.Cu") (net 8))
 (segment (start 158.700996 115) (end 157.656497 115) (width 0.25) (layer "F.Cu") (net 8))
 (segment (start 173.8875 124.4) (end 172.6875 123.2) (width 0.25) (layer "F.Cu") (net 12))
 (segment (start 167.235 121.375) (end 167.235 119.765) (width 0.25) (layer "F.Cu") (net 12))
 (segment (start 167.235 119.765) (end 168.5 118.5) (width 0.25) (layer "F.Cu") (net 12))
 (segment (start 172.6875 123.2) (end 172.1 123.2) (width 0.25) (layer "F.Cu") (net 12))
 (via (at 168.5 118.5) (size 0.8) (drill 0.4) (layers "F.Cu" "B.Cu") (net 12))
 (via (at 172.1 123.2) (size 0.8) (drill 0.4) (layers "F.Cu" "B.Cu") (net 12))
 (segment (start 168.5 118.5) (end 172.1 122.1) (width 0.25) (layer "B.Cu") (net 12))
 (segment (start 172.1 122.1) (end 172.1 123.2) (width 0.25) (layer "B.Cu") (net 12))
 (segment (start 172.3125 124.4) (end 170.7875 124.4) (width 0.25) (layer "F.Cu") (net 2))
 (segment (start 157.681596 118.035149) (end 157.681596 118.718404) (width 0.25) (layer "F.Cu") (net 6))
 (segment (start 157.494975 117.848528) (end 157.681596 118.035149) (width 0.25) (layer "F.Cu") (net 6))
 (segment (start 157.681596 118.718404) (end 156.4 120) (width 0.25) (layer "F.Cu") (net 6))
 (segment (start 163.1 119.1) (end 163.1 120) (width 0.25) (layer "F.Cu") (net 7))
 (segment (start 161.175024 117.175024) (end 163.1 119.1) (width 0.25) (layer "F.Cu") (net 7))
 (segment (start 158.035149 117.681596) (end 158.618404 117.681596) (width 0.25) (layer "F.Cu") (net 7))
 (segment (start 158.618404 117.681596) (end 159.124976 117.175024) (width 0.25) (layer "F.Cu") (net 7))
 (segment (start 157.848528 117.494975) (end 158.035149 117.681596) (width 0.25) (layer "F.Cu") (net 7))
 (segment (start 159.124976 117.175024) (end 161.175024 117.175024) (width 0.25) (layer "F.Cu") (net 7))
 (segment (start 165.965 120.080391) (end 166.896916 119.148475) (width 0.25) (layer "F.Cu") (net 11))
 (segment (start 165.965 121.375) (end 165.965 120.080391) (width 0.25) (layer "F.Cu") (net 11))
 (via (at 166.896916 119.148475) (size 0.8) (drill 0.4) (layers "F.Cu" "B.Cu") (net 11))
 (segment (start 167.9 121.65) (end 166.896916 120.646916) (width 0.25) (layer "B.Cu") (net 11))
 (segment (start 166.896916 120.646916) (end 166.896916 119.148475) (width 0.25) (layer "B.Cu") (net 11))
 (segment (start 166.24001 115.17499) (end 170.04999 115.17499) (width 0.25) (layer "F.Cu") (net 13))
 (segment (start 170.04999 115.17499) (end 170.575 115.7) (width 0.25) (layer "F.Cu") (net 13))
 (segment (start 165.965 115.45) (end 166.24001 115.17499) (width 0.25) (layer "F.Cu") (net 13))
 (segment (start 165.965 116.425) (end 165.965 115.45) (width 0.25) (layer "F.Cu") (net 13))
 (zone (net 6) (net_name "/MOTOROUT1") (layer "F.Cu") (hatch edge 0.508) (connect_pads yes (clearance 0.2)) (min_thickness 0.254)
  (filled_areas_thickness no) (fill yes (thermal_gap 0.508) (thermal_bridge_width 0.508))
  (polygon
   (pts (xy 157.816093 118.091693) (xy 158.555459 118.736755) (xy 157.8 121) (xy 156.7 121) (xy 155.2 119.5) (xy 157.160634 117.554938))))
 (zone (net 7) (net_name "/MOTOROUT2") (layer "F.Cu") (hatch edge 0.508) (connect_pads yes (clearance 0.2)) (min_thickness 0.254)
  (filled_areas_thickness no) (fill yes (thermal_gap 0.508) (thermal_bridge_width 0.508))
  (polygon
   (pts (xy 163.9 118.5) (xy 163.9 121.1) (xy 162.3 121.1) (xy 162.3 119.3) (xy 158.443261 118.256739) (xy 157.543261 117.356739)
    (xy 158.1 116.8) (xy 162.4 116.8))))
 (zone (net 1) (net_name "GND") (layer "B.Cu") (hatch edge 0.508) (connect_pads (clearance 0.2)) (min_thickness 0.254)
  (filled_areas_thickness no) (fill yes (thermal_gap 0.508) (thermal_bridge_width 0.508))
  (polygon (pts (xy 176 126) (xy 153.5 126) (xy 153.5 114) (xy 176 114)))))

